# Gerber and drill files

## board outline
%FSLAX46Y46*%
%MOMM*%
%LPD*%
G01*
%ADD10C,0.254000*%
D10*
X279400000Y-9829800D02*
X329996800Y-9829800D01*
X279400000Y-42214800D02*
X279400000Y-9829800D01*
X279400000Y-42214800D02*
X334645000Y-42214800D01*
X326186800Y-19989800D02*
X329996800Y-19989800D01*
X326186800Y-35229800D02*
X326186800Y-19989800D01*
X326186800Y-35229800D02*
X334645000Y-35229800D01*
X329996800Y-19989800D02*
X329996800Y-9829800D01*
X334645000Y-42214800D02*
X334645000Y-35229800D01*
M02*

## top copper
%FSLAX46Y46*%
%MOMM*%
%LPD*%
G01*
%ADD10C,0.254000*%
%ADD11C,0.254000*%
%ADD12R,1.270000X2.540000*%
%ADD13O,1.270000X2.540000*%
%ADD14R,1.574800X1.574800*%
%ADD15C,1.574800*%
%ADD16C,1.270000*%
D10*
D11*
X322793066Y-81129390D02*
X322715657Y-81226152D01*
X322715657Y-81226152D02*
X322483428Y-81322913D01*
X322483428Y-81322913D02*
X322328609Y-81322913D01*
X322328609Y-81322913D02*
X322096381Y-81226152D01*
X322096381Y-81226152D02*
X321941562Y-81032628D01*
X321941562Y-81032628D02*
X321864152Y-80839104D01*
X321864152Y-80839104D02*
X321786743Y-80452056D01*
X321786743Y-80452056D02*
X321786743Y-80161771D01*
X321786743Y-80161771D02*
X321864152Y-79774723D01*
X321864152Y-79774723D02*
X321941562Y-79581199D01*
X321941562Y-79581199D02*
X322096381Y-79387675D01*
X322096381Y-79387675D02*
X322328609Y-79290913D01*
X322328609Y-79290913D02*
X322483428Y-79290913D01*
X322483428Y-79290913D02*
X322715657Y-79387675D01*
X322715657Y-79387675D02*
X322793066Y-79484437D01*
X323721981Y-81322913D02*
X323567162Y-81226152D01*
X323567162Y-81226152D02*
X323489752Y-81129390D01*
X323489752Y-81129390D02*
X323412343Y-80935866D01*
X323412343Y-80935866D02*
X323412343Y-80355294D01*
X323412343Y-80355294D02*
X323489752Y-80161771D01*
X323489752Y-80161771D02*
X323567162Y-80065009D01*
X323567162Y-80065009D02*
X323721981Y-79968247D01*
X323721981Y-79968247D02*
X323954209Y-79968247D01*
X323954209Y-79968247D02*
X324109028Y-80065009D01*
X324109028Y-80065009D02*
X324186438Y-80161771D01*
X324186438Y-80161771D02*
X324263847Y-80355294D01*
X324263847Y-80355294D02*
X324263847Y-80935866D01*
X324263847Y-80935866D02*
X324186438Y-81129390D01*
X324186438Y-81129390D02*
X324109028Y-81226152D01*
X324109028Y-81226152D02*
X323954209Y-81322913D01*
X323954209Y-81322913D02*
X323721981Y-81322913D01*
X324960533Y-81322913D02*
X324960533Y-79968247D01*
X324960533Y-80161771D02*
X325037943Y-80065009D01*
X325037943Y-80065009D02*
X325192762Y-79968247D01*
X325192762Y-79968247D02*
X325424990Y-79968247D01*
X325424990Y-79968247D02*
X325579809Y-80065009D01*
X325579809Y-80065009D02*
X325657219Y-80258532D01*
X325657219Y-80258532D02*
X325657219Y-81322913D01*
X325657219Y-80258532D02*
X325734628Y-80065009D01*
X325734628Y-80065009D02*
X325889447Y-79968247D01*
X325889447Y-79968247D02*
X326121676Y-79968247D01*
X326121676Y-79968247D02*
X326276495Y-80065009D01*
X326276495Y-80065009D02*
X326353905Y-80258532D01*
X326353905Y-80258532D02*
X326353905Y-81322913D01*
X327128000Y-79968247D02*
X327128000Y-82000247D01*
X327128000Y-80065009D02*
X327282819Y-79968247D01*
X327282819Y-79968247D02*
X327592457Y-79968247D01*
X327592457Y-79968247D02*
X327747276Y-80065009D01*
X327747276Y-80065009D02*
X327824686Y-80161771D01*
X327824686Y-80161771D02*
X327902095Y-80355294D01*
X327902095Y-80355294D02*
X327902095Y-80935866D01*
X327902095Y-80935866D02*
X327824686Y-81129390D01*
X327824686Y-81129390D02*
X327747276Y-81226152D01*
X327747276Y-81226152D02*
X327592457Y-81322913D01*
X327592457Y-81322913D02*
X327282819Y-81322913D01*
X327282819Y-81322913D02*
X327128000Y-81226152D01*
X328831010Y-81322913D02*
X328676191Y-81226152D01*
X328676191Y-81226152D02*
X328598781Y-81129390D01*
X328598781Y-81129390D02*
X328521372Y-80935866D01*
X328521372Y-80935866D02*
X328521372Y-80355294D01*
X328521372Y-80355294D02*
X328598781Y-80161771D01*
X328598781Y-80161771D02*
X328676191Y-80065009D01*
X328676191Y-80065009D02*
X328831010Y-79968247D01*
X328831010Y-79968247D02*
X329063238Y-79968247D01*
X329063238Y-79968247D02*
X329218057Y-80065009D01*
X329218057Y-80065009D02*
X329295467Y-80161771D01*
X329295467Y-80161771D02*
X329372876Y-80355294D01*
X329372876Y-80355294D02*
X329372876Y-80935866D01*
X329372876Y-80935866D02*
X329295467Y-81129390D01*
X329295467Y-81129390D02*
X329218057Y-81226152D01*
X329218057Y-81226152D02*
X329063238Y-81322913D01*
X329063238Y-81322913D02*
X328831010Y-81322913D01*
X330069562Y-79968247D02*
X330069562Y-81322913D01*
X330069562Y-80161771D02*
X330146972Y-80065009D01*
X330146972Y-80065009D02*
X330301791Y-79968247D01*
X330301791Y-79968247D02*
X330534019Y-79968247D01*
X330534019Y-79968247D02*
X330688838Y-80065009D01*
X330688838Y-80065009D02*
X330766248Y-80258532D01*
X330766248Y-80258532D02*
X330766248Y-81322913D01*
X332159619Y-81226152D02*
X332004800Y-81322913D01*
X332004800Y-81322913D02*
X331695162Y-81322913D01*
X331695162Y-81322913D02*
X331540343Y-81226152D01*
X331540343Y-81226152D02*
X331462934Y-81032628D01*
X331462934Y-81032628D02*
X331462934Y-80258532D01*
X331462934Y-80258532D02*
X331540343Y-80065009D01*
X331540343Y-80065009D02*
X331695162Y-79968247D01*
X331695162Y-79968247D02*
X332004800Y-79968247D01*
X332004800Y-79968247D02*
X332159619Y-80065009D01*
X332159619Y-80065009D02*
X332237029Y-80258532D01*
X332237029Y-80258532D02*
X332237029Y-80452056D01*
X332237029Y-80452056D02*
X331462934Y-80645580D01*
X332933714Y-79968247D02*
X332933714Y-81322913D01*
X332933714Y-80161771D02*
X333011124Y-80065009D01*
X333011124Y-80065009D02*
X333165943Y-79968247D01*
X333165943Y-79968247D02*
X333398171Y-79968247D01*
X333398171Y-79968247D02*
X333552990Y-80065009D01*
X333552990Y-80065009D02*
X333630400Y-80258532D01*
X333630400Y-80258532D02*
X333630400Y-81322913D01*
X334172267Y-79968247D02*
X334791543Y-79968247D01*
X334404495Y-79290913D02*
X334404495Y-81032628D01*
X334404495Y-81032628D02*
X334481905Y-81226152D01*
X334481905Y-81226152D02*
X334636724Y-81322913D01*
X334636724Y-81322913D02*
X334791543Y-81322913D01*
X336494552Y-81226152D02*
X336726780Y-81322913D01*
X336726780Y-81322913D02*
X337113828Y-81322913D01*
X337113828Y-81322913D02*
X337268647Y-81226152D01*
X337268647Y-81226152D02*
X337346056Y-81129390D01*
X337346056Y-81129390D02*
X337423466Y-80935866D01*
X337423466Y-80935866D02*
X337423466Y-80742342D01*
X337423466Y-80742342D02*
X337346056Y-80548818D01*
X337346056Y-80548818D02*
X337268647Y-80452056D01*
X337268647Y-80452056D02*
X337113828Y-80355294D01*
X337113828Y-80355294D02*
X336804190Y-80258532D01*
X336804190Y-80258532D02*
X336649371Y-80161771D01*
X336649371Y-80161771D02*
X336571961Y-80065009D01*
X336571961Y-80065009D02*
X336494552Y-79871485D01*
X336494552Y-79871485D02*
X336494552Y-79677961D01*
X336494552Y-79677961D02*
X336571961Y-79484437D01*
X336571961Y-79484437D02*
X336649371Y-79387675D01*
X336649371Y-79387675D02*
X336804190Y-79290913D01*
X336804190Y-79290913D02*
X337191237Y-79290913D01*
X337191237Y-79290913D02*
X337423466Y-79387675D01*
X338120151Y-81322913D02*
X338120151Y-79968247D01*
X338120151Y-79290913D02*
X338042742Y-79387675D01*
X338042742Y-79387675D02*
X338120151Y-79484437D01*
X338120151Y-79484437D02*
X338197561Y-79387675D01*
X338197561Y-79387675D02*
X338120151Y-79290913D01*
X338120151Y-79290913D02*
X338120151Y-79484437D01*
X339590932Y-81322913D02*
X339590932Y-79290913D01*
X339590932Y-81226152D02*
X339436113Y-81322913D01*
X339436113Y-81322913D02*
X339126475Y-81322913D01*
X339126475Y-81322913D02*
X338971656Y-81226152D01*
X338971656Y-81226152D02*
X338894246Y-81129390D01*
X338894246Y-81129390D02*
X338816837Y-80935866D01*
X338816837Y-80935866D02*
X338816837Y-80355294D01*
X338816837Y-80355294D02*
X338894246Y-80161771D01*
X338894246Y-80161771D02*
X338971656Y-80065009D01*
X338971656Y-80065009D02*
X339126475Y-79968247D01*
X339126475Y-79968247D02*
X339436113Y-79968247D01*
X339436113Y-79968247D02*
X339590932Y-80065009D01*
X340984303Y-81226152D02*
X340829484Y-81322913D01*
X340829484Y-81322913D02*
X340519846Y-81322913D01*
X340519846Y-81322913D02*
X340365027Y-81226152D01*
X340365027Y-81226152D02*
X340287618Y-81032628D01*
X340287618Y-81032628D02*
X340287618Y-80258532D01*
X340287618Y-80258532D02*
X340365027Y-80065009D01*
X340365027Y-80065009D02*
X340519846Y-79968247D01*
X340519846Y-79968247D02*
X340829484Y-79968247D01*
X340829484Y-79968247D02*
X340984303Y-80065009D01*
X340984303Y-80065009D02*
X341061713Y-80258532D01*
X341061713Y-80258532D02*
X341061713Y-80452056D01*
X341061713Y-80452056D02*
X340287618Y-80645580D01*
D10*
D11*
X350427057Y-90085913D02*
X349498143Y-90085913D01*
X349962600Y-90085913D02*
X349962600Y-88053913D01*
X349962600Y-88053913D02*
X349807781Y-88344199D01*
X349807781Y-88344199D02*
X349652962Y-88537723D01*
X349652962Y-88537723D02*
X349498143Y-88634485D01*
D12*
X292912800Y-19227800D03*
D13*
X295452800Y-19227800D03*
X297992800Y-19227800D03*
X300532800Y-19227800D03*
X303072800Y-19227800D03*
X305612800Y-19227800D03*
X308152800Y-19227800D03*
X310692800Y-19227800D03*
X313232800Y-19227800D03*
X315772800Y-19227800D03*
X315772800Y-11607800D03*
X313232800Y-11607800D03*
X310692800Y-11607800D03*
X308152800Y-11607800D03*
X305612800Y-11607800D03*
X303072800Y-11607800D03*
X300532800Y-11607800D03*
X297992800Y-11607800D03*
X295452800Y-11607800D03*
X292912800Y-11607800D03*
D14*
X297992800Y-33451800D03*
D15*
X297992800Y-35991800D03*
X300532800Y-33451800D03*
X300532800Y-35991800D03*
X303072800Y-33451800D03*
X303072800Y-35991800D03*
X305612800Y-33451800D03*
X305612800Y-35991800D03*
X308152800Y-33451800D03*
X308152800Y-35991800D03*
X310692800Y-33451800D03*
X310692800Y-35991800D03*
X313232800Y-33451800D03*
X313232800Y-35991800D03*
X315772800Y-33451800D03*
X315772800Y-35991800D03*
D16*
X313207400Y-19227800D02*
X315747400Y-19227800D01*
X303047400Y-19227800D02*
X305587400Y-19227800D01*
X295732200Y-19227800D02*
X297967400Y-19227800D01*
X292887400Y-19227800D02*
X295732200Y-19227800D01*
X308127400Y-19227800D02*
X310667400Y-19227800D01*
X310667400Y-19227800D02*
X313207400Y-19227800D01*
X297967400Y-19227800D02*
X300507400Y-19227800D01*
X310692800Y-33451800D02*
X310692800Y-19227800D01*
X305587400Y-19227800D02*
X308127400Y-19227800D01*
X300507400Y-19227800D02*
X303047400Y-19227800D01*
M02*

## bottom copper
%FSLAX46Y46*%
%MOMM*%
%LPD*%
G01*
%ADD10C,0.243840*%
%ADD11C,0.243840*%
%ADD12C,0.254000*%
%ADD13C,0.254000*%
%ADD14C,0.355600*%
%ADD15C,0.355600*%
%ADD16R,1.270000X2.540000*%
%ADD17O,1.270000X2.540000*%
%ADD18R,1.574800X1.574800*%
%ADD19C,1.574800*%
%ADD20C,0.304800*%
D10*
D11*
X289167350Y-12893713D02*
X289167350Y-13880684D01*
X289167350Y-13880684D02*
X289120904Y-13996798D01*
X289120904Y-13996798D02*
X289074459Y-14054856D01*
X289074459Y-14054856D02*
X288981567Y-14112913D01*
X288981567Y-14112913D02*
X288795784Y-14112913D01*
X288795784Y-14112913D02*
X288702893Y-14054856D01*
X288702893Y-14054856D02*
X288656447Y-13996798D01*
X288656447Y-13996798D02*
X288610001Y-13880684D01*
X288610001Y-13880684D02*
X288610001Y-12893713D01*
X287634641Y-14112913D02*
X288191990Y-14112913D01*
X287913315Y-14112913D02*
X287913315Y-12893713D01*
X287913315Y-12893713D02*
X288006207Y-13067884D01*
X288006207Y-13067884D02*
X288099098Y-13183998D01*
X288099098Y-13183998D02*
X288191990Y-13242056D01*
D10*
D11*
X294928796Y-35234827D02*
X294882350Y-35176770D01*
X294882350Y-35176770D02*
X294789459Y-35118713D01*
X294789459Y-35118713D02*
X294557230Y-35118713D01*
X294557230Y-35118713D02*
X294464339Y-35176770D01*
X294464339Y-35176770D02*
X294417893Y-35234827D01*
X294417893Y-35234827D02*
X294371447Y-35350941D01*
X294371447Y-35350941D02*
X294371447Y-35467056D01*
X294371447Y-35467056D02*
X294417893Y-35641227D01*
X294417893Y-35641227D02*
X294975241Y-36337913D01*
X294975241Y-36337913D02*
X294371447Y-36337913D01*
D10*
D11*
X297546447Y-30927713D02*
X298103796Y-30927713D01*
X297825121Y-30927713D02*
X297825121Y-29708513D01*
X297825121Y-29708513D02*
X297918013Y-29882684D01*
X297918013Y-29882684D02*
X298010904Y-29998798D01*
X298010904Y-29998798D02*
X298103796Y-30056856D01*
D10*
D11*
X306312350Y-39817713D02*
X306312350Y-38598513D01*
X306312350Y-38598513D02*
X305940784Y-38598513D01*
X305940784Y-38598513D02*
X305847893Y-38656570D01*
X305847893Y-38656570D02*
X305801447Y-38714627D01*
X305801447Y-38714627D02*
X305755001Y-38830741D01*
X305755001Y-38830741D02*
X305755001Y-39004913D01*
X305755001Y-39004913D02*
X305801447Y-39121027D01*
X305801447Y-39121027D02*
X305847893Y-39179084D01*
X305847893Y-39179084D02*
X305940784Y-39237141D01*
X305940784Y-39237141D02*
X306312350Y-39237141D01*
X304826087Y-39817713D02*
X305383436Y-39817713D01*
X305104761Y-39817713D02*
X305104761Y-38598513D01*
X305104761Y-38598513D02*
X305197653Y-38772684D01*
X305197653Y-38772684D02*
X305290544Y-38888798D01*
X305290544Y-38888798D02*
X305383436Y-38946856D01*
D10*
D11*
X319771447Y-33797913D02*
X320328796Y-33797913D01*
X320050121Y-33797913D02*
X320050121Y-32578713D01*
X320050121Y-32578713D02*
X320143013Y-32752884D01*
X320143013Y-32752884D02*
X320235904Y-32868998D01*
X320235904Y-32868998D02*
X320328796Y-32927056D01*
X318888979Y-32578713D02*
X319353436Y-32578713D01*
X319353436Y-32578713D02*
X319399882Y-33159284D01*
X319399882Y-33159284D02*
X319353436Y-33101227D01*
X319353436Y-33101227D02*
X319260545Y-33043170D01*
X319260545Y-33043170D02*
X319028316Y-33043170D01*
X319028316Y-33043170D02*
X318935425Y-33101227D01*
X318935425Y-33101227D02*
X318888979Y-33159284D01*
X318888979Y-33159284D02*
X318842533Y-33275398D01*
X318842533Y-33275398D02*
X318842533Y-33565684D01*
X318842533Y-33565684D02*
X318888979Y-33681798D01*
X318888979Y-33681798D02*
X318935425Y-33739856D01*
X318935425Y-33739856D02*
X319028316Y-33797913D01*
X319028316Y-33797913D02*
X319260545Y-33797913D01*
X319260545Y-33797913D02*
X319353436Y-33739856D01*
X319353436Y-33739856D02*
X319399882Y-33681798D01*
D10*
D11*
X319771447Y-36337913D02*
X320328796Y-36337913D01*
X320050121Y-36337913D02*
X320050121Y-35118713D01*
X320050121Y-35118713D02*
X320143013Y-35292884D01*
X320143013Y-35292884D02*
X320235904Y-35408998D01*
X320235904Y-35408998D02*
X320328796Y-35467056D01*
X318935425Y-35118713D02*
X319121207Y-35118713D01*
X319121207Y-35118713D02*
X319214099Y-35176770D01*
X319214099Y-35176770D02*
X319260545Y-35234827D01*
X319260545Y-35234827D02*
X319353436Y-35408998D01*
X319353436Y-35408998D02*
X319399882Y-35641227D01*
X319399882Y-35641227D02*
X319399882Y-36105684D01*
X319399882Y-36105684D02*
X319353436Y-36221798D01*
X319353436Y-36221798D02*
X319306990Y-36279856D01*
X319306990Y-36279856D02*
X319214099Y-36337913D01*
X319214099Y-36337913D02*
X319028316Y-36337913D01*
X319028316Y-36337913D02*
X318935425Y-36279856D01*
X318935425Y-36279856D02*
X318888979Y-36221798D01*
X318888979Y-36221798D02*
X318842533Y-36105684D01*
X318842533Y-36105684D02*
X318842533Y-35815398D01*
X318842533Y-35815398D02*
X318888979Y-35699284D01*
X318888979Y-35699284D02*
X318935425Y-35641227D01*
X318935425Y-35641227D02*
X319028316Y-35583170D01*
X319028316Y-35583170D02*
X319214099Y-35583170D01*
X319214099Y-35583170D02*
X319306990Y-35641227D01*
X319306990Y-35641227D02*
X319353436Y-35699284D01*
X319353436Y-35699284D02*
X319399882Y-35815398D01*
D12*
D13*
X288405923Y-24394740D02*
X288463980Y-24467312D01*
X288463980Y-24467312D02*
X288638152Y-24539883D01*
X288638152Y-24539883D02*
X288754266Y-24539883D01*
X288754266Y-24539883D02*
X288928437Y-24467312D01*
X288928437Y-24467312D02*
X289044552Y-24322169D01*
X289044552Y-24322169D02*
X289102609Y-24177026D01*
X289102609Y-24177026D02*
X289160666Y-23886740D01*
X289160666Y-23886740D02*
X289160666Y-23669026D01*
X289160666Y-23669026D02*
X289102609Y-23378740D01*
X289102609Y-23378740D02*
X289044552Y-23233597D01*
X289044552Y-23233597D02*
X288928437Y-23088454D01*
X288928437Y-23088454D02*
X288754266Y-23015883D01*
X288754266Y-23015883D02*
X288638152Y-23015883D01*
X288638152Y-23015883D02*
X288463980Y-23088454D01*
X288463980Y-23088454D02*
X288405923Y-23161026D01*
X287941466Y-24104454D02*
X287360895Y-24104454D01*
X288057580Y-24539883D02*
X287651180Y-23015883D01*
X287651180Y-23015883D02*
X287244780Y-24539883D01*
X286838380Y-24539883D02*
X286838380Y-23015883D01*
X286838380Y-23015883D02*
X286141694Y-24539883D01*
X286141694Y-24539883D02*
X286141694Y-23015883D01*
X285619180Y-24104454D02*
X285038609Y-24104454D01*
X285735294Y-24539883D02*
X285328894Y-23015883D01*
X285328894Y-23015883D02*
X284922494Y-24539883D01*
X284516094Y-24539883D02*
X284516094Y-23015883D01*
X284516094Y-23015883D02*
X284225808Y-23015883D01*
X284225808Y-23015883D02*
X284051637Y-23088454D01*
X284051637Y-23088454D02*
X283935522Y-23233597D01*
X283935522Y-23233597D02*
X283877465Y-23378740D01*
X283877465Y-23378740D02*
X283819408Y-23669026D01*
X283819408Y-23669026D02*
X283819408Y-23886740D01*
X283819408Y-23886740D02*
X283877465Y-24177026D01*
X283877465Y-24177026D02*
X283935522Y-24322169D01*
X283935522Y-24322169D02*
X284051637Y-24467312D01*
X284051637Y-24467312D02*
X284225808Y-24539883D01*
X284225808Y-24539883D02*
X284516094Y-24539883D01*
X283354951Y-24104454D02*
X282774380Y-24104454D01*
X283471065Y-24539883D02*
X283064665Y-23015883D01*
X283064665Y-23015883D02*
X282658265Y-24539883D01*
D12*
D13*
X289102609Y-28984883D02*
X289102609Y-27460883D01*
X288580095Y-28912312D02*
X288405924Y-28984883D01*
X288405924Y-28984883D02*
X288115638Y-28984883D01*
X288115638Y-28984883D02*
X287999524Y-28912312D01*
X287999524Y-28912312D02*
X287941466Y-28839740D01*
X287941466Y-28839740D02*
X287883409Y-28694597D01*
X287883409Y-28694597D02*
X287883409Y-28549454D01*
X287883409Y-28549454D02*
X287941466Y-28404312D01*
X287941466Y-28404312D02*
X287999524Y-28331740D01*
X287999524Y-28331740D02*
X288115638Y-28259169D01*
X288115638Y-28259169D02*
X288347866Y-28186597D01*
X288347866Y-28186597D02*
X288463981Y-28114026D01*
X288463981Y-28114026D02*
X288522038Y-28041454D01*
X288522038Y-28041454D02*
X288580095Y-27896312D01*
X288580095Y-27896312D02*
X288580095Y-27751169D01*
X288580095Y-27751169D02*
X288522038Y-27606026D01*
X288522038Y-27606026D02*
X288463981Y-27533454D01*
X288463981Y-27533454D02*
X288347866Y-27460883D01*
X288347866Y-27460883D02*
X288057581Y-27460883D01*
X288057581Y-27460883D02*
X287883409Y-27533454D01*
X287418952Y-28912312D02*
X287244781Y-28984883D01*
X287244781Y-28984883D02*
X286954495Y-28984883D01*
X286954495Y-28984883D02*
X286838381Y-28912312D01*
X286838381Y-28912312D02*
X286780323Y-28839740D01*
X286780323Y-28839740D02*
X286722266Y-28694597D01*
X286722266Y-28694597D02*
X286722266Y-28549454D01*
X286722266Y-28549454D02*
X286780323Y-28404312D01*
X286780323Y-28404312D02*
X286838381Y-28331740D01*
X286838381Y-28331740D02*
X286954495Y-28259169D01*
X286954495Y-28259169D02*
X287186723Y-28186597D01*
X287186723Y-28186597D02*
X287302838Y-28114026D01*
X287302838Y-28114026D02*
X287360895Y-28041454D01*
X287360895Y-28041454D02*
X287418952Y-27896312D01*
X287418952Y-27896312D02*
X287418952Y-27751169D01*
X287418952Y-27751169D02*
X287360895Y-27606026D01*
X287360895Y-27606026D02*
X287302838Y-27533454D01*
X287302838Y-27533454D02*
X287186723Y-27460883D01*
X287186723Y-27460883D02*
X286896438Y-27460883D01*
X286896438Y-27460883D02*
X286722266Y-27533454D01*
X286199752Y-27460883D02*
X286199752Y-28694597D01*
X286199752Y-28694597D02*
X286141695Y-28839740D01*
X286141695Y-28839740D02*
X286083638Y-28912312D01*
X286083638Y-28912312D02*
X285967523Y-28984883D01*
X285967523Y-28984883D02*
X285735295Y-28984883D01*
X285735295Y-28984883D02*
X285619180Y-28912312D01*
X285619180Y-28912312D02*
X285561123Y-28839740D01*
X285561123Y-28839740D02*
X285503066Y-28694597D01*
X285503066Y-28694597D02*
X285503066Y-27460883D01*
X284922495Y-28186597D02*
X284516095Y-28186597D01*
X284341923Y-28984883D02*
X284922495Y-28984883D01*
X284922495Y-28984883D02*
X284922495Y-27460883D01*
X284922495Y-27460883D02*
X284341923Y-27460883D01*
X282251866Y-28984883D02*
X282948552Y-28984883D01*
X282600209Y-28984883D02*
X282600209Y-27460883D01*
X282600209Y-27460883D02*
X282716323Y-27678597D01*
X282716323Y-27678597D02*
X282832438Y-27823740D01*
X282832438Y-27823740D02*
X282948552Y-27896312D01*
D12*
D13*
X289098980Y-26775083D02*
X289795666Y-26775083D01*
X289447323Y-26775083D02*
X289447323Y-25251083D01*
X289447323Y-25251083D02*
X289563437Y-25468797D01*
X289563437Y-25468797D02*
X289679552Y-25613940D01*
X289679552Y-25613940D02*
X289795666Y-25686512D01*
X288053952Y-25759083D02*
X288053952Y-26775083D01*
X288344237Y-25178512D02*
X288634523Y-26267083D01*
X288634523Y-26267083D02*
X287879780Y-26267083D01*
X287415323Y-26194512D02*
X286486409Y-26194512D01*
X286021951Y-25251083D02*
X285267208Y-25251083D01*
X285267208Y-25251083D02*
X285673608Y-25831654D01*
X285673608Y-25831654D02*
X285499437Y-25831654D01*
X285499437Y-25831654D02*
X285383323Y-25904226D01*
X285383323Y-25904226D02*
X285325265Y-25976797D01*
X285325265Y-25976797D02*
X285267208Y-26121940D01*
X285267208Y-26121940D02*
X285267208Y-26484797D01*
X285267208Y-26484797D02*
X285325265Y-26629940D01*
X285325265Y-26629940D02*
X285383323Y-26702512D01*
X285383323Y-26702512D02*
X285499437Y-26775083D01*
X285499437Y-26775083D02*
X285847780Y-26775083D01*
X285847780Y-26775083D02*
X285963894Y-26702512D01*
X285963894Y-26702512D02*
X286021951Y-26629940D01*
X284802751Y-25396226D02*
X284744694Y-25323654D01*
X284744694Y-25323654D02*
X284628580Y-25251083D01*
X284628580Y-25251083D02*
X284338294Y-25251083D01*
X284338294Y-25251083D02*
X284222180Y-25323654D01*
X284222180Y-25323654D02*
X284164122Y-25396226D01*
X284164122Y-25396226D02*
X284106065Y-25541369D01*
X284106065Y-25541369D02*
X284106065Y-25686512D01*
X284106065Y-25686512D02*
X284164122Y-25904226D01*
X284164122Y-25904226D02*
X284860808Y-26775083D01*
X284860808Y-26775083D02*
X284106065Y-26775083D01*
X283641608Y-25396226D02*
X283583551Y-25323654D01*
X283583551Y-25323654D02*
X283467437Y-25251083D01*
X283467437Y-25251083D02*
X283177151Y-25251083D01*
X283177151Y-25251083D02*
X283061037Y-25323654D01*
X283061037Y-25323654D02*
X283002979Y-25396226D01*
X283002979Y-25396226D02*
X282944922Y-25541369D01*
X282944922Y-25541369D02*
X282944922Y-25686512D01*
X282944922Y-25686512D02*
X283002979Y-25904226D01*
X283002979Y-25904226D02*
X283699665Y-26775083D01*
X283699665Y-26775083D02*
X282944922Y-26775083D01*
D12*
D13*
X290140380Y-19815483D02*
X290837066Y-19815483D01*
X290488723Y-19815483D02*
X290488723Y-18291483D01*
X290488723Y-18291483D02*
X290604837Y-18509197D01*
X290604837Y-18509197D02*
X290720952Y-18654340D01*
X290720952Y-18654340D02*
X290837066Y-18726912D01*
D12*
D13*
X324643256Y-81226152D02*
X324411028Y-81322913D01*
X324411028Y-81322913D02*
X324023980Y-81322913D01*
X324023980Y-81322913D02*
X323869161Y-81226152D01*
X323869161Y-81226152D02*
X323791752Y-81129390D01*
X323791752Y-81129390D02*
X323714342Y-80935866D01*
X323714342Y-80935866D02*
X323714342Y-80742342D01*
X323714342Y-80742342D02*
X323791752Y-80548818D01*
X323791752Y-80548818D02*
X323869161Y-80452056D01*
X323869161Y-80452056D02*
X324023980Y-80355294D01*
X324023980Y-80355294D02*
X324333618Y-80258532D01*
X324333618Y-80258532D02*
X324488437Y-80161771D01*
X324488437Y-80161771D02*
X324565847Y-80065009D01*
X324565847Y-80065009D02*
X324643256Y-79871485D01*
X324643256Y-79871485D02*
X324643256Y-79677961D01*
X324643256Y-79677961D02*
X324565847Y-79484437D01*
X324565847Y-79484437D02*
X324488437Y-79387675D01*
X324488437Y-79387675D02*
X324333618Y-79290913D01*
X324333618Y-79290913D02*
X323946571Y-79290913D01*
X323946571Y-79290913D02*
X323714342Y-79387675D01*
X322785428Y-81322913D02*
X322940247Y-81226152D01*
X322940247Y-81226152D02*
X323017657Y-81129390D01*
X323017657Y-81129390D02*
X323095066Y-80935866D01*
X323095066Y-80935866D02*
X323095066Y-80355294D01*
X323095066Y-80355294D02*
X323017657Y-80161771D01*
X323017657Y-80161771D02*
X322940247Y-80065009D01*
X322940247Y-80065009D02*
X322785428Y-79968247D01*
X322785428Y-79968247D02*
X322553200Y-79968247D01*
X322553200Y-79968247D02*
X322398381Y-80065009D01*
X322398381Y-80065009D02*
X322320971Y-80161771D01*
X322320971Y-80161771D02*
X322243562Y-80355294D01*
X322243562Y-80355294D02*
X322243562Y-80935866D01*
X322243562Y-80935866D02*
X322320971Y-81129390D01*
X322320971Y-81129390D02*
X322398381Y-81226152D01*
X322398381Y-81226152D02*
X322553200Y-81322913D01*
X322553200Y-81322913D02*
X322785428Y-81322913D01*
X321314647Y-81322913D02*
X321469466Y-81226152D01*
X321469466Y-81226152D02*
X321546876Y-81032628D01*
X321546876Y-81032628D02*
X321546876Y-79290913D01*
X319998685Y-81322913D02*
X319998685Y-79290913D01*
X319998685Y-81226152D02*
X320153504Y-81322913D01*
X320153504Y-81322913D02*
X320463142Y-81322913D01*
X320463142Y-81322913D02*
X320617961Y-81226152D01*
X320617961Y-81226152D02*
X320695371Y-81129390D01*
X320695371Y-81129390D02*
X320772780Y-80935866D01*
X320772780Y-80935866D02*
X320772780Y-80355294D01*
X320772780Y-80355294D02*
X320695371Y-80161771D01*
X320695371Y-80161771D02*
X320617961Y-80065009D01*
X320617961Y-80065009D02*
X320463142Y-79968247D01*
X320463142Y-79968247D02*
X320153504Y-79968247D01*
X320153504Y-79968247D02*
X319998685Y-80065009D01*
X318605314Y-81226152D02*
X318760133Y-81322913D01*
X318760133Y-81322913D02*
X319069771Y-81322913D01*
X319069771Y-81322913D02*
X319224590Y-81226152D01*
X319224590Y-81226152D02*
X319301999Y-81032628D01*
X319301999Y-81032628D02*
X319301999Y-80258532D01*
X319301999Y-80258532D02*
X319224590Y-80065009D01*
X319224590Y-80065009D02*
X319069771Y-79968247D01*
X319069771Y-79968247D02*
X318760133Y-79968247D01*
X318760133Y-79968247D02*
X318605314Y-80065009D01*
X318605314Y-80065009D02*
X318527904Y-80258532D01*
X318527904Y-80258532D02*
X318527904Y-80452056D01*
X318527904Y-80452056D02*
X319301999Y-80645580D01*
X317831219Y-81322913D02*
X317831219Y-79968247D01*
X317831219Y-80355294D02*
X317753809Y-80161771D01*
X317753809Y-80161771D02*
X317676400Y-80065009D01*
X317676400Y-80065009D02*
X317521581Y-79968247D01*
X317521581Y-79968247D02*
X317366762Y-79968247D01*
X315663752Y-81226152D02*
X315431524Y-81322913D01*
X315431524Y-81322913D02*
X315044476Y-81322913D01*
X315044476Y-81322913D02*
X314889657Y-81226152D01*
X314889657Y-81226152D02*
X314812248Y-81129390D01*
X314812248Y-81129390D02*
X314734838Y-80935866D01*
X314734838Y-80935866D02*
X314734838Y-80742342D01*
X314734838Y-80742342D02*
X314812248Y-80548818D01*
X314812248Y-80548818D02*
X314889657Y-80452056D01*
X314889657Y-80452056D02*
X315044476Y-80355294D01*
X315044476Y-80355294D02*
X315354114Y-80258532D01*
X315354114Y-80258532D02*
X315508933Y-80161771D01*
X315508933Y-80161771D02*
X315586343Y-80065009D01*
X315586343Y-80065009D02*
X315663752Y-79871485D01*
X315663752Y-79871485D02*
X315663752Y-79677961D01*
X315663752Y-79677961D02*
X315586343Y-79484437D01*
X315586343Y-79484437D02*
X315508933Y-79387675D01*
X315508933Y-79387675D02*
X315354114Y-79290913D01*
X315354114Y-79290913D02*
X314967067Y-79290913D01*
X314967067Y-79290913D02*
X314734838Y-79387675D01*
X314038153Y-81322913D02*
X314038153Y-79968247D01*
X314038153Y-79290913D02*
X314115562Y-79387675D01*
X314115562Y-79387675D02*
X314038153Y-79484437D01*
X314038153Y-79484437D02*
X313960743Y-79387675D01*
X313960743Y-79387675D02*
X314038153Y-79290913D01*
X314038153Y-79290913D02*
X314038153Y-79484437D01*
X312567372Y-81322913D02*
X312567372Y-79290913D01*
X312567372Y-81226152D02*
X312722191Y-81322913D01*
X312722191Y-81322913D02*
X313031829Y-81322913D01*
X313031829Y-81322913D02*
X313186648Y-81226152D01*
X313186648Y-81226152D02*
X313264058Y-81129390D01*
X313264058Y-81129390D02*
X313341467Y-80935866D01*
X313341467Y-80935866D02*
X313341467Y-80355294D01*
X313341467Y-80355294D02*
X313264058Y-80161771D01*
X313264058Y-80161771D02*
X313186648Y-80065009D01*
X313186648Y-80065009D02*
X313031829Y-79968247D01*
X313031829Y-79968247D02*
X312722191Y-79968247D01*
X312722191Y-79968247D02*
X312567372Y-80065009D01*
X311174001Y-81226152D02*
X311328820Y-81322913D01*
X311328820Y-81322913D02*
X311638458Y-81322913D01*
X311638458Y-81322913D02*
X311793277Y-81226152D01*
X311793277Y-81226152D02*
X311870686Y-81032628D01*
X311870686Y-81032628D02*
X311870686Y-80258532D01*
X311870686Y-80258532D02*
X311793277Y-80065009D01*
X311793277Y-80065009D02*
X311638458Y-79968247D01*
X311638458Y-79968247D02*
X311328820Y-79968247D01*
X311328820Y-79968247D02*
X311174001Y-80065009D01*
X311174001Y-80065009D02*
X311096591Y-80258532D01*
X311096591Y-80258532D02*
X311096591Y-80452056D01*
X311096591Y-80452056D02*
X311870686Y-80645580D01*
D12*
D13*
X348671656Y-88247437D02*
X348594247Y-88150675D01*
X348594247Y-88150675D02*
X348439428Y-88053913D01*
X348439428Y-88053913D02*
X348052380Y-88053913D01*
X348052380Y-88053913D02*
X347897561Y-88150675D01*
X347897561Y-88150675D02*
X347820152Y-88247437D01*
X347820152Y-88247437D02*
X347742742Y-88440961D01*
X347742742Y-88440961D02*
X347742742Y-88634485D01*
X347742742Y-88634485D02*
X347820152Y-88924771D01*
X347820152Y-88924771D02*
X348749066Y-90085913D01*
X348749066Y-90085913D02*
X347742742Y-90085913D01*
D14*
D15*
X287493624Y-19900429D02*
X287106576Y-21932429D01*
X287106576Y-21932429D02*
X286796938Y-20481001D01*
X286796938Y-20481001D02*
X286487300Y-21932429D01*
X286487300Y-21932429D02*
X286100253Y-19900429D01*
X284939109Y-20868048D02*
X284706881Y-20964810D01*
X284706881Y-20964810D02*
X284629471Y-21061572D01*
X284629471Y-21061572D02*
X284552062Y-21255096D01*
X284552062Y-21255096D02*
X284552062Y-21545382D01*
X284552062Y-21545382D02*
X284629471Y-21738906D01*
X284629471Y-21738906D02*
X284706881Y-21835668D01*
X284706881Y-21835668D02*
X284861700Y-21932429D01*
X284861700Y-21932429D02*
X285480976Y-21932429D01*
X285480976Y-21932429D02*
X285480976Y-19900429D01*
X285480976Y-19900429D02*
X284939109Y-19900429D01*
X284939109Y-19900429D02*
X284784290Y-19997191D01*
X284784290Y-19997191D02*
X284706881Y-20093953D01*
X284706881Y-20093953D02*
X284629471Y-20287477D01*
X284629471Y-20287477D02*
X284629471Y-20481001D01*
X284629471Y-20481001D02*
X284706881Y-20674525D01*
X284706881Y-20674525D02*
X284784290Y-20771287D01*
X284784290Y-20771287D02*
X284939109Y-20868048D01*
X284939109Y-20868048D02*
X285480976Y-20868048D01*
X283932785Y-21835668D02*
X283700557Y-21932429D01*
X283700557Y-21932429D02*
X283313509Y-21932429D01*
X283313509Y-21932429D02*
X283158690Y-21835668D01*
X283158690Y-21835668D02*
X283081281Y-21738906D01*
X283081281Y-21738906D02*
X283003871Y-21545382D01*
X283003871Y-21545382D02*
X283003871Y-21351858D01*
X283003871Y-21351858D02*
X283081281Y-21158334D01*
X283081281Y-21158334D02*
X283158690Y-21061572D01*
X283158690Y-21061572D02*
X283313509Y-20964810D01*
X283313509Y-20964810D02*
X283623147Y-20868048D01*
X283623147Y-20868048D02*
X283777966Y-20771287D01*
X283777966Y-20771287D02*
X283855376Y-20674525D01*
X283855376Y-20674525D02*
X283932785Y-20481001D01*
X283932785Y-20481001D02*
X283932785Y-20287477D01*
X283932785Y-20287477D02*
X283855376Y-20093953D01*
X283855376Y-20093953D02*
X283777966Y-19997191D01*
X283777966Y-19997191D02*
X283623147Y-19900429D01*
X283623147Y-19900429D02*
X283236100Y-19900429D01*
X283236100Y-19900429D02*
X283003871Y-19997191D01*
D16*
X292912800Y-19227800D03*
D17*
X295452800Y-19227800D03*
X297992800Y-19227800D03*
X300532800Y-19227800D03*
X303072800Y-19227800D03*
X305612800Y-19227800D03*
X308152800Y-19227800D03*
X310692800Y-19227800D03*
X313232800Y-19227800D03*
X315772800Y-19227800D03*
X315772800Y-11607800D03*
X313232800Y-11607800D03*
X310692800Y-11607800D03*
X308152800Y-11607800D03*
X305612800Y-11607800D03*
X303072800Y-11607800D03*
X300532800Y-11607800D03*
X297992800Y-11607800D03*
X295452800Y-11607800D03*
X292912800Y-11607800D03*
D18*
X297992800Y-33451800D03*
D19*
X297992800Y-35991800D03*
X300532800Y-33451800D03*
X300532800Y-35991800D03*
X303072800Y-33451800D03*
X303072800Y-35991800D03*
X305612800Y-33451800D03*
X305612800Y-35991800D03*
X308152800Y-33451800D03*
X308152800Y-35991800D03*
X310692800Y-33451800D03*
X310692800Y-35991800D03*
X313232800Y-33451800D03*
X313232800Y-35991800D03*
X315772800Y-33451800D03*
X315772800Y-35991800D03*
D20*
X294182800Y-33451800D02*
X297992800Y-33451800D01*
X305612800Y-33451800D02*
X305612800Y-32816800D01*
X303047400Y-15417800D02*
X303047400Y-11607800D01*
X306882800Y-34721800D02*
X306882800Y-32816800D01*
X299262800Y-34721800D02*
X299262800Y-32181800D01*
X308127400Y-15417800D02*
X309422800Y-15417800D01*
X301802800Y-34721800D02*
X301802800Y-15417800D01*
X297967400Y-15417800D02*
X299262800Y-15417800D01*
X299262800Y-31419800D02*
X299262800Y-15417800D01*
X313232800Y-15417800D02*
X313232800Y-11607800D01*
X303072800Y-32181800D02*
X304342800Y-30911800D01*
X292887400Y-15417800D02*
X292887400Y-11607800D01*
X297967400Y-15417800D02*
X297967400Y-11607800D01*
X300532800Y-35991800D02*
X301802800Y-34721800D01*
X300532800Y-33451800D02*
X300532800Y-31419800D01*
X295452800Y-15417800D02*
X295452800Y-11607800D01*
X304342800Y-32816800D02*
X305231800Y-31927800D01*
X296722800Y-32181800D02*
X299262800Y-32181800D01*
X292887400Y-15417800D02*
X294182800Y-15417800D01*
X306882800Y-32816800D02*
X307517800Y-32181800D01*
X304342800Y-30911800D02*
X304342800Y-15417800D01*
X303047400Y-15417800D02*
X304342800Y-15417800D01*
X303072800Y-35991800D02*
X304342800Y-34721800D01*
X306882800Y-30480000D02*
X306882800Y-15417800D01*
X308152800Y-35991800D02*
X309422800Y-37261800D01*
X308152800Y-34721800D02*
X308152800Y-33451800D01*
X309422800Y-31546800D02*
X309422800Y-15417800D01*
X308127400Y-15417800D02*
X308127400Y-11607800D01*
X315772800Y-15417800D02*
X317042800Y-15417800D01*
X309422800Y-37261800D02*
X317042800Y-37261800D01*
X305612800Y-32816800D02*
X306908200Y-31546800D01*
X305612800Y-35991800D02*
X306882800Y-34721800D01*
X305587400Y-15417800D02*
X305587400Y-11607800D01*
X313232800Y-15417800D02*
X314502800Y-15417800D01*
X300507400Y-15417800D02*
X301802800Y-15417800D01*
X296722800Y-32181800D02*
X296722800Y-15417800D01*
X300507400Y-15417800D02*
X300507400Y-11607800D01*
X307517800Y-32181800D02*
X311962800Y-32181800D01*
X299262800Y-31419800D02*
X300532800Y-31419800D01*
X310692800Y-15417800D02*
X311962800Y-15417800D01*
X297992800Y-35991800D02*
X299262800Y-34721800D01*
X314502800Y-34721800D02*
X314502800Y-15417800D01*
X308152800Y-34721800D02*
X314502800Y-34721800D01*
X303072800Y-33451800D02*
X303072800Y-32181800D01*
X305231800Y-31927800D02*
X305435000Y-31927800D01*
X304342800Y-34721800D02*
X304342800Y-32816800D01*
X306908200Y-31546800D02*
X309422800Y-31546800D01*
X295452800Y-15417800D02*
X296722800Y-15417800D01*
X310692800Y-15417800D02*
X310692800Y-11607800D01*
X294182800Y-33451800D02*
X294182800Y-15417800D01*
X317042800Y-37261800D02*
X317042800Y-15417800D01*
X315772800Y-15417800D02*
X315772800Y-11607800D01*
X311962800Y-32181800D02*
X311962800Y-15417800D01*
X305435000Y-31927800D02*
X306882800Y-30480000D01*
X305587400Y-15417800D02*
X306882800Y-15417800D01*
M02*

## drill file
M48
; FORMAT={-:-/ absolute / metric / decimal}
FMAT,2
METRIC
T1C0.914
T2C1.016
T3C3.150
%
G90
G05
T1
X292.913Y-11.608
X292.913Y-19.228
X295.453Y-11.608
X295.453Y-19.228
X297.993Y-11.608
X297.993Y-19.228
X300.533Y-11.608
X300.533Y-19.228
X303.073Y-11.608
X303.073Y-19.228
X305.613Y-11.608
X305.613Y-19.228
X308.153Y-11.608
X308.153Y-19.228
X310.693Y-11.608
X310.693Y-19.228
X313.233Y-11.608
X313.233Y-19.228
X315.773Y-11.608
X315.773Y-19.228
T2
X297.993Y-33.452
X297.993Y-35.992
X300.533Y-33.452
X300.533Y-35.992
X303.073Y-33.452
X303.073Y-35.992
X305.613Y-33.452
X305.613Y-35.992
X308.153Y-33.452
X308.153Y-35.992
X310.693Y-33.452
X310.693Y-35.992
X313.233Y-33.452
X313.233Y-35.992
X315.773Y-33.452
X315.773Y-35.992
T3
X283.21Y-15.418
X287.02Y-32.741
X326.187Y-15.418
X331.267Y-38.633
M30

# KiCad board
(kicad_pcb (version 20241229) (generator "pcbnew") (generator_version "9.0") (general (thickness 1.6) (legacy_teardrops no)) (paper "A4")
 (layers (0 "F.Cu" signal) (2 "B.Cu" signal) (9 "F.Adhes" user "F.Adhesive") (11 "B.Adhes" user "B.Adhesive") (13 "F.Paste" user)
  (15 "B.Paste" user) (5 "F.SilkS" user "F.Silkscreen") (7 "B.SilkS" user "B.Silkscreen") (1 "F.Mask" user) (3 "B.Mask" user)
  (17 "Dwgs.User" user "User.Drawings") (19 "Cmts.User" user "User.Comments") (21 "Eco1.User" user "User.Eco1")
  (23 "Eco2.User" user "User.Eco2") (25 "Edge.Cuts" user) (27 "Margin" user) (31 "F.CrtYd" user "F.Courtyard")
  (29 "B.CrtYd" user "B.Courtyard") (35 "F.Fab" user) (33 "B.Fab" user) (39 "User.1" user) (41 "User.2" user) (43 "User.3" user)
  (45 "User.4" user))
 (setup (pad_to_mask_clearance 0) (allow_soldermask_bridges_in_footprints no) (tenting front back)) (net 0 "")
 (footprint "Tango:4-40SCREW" (layer "F.Cu") (at 287.02 32.7406)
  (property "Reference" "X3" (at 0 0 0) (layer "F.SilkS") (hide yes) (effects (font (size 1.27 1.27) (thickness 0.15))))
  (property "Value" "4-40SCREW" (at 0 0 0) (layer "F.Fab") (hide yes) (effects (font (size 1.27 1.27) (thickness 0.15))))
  (pad "" np_thru_hole circle (at 0 0) (size 3.1496 3.1496) (drill 3.1496) (layers "*.Cu" "*.Mask")))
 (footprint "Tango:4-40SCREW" (layer "F.Cu") (at 283.21 15.4178)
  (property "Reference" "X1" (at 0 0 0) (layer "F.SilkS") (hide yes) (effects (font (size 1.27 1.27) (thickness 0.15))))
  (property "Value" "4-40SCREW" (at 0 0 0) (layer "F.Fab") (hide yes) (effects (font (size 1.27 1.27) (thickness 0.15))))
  (pad "" np_thru_hole circle (at 0 0) (size 3.1496 3.1496) (drill 3.1496) (layers "*.Cu" "*.Mask")))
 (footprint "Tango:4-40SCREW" (layer "F.Cu") (at 331.2668 38.6334)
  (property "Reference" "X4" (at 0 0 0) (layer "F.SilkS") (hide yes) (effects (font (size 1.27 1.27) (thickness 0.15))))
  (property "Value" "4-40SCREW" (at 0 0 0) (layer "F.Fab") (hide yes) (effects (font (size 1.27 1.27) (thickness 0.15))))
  (pad "" np_thru_hole circle (at 0 0) (size 3.1496 3.1496) (drill 3.1496) (layers "*.Cu" "*.Mask")))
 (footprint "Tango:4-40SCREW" (layer "F.Cu") (at 326.1868 15.4178)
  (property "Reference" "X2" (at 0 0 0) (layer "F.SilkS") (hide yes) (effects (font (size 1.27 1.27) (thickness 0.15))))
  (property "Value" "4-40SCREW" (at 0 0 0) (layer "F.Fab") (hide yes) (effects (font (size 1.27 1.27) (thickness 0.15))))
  (pad "" np_thru_hole circle (at 0 0) (size 3.1496 3.1496) (drill 3.1496) (layers "*.Cu" "*.Mask")))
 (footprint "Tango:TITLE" (layer "F.Cu") (at 370.84 91.1098)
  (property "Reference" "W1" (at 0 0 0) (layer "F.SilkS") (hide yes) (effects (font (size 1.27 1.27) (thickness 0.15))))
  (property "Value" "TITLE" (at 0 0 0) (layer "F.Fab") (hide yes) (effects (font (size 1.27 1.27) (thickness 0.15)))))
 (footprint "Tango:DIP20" (layer "F.Cu") (at 292.9128 19.2278)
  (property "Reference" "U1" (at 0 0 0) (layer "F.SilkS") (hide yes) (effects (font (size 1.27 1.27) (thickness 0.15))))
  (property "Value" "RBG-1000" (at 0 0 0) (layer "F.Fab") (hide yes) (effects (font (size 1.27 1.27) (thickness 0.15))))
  (pad "1" thru_hole rect (at 0 0) (size 1.27 2.54) (drill 0.9144) (layers "*.Cu" "*.Mask") (remove_unused_layers no)
   (thermal_bridge_angle 45))
  (pad "2" thru_hole oval (at 2.54 0) (size 1.27 2.54) (drill 0.9144) (layers "*.Cu" "*.Mask") (remove_unused_layers no)
   (thermal_bridge_angle 45))
  (pad "3" thru_hole oval (at 5.08 0) (size 1.27 2.54) (drill 0.9144) (layers "*.Cu" "*.Mask") (remove_unused_layers no)
   (thermal_bridge_angle 45))
  (pad "4" thru_hole oval (at 7.62 0) (size 1.27 2.54) (drill 0.9144) (layers "*.Cu" "*.Mask") (remove_unused_layers no)
   (thermal_bridge_angle 45))
  (pad "5" thru_hole oval (at 10.16 0) (size 1.27 2.54) (drill 0.9144) (layers "*.Cu" "*.Mask") (remove_unused_layers no)
   (thermal_bridge_angle 45))
  (pad "6" thru_hole oval (at 12.7 0) (size 1.27 2.54) (drill 0.9144) (layers "*.Cu" "*.Mask") (remove_unused_layers no)
   (thermal_bridge_angle 45))
  (pad "7" thru_hole oval (at 15.24 0) (size 1.27 2.54) (drill 0.9144) (layers "*.Cu" "*.Mask") (remove_unused_layers no)
   (thermal_bridge_angle 45))
  (pad "8" thru_hole oval (at 17.78 0) (size 1.27 2.54) (drill 0.9144) (layers "*.Cu" "*.Mask") (remove_unused_layers no)
   (thermal_bridge_angle 45))
  (pad "9" thru_hole oval (at 20.32 0) (size 1.27 2.54) (drill 0.9144) (layers "*.Cu" "*.Mask") (remove_unused_layers no)
   (thermal_bridge_angle 45))
  (pad "10" thru_hole oval (at 22.86 0) (size 1.27 2.54) (drill 0.9144) (layers "*.Cu" "*.Mask") (remove_unused_layers no)
   (thermal_bridge_angle 45))
  (pad "11" thru_hole oval (at 22.86 -7.62) (size 1.27 2.54) (drill 0.9144) (layers "*.Cu" "*.Mask") (remove_unused_layers no)
   (thermal_bridge_angle 45))
  (pad "12" thru_hole oval (at 20.32 -7.62) (size 1.27 2.54) (drill 0.9144) (layers "*.Cu" "*.Mask") (remove_unused_layers no)
   (thermal_bridge_angle 45))
  (pad "13" thru_hole oval (at 17.78 -7.62) (size 1.27 2.54) (drill 0.9144) (layers "*.Cu" "*.Mask") (remove_unused_layers no)
   (thermal_bridge_angle 45))
  (pad "14" thru_hole oval (at 15.24 -7.62) (size 1.27 2.54) (drill 0.9144) (layers "*.Cu" "*.Mask") (remove_unused_layers no)
   (thermal_bridge_angle 45))
  (pad "15" thru_hole oval (at 12.7 -7.62) (size 1.27 2.54) (drill 0.9144) (layers "*.Cu" "*.Mask") (remove_unused_layers no)
   (thermal_bridge_angle 45))
  (pad "16" thru_hole oval (at 10.16 -7.62) (size 1.27 2.54) (drill 0.9144) (layers "*.Cu" "*.Mask") (remove_unused_layers no)
   (thermal_bridge_angle 45))
  (pad "17" thru_hole oval (at 7.62 -7.62) (size 1.27 2.54) (drill 0.9144) (layers "*.Cu" "*.Mask") (remove_unused_layers no)
   (thermal_bridge_angle 45))
  (pad "18" thru_hole oval (at 5.08 -7.62) (size 1.27 2.54) (drill 0.9144) (layers "*.Cu" "*.Mask") (remove_unused_layers no)
   (thermal_bridge_angle 45))
  (pad "19" thru_hole oval (at 2.54 -7.62) (size 1.27 2.54) (drill 0.9144) (layers "*.Cu" "*.Mask") (remove_unused_layers no)
   (thermal_bridge_angle 45))
  (pad "20" thru_hole oval (at 0 -7.62) (size 1.27 2.54) (drill 0.9144) (layers "*.Cu" "*.Mask") (remove_unused_layers no)
   (thermal_bridge_angle 45)))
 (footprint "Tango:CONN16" (layer "F.Cu") (at 297.9928 35.9918)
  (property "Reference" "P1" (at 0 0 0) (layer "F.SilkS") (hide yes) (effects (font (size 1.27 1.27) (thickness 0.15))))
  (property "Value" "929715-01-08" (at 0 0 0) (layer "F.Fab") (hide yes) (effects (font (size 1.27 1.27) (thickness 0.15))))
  (pad "1" thru_hole rect (at 0 -2.54) (size 1.5748 1.5748) (drill 1.016) (layers "*.Cu" "*.Mask") (remove_unused_layers no)
   (thermal_bridge_angle 45))
  (pad "2" thru_hole circle (at 0 0) (size 1.5748 1.5748) (drill 1.016) (layers "*.Cu" "*.Mask") (remove_unused_layers no))
  (pad "3" thru_hole circle (at 2.54 -2.54) (size 1.5748 1.5748) (drill 1.016) (layers "*.Cu" "*.Mask") (remove_unused_layers no))
  (pad "4" thru_hole circle (at 2.54 0) (size 1.5748 1.5748) (drill 1.016) (layers "*.Cu" "*.Mask") (remove_unused_layers no))
  (pad "5" thru_hole circle (at 5.08 -2.54) (size 1.5748 1.5748) (drill 1.016) (layers "*.Cu" "*.Mask") (remove_unused_layers no))
  (pad "6" thru_hole circle (at 5.08 0) (size 1.5748 1.5748) (drill 1.016) (layers "*.Cu" "*.Mask") (remove_unused_layers no))
  (pad "7" thru_hole circle (at 7.62 -2.54) (size 1.5748 1.5748) (drill 1.016) (layers "*.Cu" "*.Mask") (remove_unused_layers no))
  (pad "8" thru_hole circle (at 7.62 0) (size 1.5748 1.5748) (drill 1.016) (layers "*.Cu" "*.Mask") (remove_unused_layers no))
  (pad "9" thru_hole circle (at 10.16 -2.54) (size 1.5748 1.5748) (drill 1.016) (layers "*.Cu" "*.Mask") (remove_unused_layers no))
  (pad "10" thru_hole circle (at 10.16 0) (size 1.5748 1.5748) (drill 1.016) (layers "*.Cu" "*.Mask") (remove_unused_layers no))
  (pad "11" thru_hole circle (at 12.7 -2.54) (size 1.5748 1.5748) (drill 1.016) (layers "*.Cu" "*.Mask") (remove_unused_layers no))
  (pad "12" thru_hole circle (at 12.7 0) (size 1.5748 1.5748) (drill 1.016) (layers "*.Cu" "*.Mask") (remove_unused_layers no))
  (pad "13" thru_hole circle (at 15.24 -2.54) (size 1.5748 1.5748) (drill 1.016) (layers "*.Cu" "*.Mask") (remove_unused_layers no))
  (pad "14" thru_hole circle (at 15.24 0) (size 1.5748 1.5748) (drill 1.016) (layers "*.Cu" "*.Mask") (remove_unused_layers no))
  (pad "15" thru_hole circle (at 17.78 -2.54) (size 1.5748 1.5748) (drill 1.016) (layers "*.Cu" "*.Mask") (remove_unused_layers no))
  (pad "16" thru_hole circle (at 17.78 0) (size 1.5748 1.5748) (drill 1.016) (layers "*.Cu" "*.Mask") (remove_unused_layers no)))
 (gr_line (start 279.4 9.8298) (end 329.9968 9.8298) (stroke (width 0.254) (type default)) (layer "Edge.Cuts"))
 (gr_line (start 279.4 42.2148) (end 279.4 9.8298) (stroke (width 0.254) (type default)) (layer "Edge.Cuts"))
 (gr_line (start 279.4 42.2148) (end 334.645 42.2148) (stroke (width 0.254) (type default)) (layer "Edge.Cuts"))
 (gr_line (start 326.1868 19.9898) (end 329.9968 19.9898) (stroke (width 0.254) (type default)) (layer "Edge.Cuts"))
 (gr_line (start 326.1868 35.2298) (end 326.1868 19.9898) (stroke (width 0.254) (type default)) (layer "Edge.Cuts"))
 (gr_line (start 326.1868 35.2298) (end 334.645 35.2298) (stroke (width 0.254) (type default)) (layer "Edge.Cuts"))
 (gr_line (start 329.9968 19.9898) (end 329.9968 9.8298) (stroke (width 0.254) (type default)) (layer "Edge.Cuts"))
 (gr_line (start 334.645 42.2148) (end 334.645 35.2298) (stroke (width 0.254) (type default)) (layer "Edge.Cuts"))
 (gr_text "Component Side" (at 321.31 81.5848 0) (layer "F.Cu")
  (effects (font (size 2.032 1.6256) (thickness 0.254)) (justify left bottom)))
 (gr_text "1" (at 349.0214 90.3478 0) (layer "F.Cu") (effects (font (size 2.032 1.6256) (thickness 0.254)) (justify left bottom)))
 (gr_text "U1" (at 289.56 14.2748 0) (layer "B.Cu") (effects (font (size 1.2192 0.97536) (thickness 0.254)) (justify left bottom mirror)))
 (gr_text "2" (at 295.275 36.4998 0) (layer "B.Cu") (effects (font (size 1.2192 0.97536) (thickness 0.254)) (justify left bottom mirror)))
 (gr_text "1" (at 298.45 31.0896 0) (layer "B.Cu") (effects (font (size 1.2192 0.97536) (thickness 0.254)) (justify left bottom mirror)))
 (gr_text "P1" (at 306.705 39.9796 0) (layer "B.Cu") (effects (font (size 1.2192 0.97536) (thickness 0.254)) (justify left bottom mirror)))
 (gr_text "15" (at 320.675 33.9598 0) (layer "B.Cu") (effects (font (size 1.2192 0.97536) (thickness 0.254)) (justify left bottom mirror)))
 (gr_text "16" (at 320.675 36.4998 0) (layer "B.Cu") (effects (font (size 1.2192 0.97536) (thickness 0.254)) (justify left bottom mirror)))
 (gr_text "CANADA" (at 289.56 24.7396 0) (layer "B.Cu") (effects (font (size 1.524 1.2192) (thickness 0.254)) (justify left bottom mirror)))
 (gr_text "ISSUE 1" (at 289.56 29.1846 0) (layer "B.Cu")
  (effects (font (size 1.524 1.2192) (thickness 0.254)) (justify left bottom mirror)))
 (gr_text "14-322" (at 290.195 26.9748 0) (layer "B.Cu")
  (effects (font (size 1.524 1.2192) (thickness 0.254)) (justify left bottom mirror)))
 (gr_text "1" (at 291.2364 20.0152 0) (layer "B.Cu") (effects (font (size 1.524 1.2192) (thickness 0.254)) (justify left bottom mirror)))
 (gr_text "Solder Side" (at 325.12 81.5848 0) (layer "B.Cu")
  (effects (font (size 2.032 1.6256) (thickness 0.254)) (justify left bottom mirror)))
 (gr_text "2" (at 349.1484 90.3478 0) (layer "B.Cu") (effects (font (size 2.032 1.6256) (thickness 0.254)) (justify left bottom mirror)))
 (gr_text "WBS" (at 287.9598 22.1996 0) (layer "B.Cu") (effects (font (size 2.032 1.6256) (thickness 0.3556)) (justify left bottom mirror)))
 (segment (start 313.2074 19.2278) (end 315.7474 19.2278) (width 1.27) (layer "F.Cu") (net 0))
 (segment (start 303.0474 19.2278) (end 305.5874 19.2278) (width 1.27) (layer "F.Cu") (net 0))
 (segment (start 295.7322 19.2278) (end 297.9674 19.2278) (width 1.27) (layer "F.Cu") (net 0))
 (segment (start 292.8874 19.2278) (end 295.7322 19.2278) (width 1.27) (layer "F.Cu") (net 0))
 (segment (start 308.1274 19.2278) (end 310.6674 19.2278) (width 1.27) (layer "F.Cu") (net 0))
 (segment (start 310.6674 19.2278) (end 313.2074 19.2278) (width 1.27) (layer "F.Cu") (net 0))
 (segment (start 297.9674 19.2278) (end 300.5074 19.2278) (width 1.27) (layer "F.Cu") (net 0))
 (segment (start 310.6928 33.4518) (end 310.6928 19.2278) (width 1.27) (layer "F.Cu") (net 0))
 (segment (start 305.5874 19.2278) (end 308.1274 19.2278) (width 1.27) (layer "F.Cu") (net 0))
 (segment (start 300.5074 19.2278) (end 303.0474 19.2278) (width 1.27) (layer "F.Cu") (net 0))
 (segment (start 294.1828 33.4518) (end 297.9928 33.4518) (width 0.3048) (layer "B.Cu") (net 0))
 (segment (start 305.6128 33.4518) (end 305.6128 32.8168) (width 0.3048) (layer "B.Cu") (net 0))
 (segment (start 303.0474 15.4178) (end 303.0474 11.6078) (width 0.3048) (layer "B.Cu") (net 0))
 (segment (start 306.8828 34.7218) (end 306.8828 32.8168) (width 0.3048) (layer "B.Cu") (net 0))
 (segment (start 299.2628 34.7218) (end 299.2628 32.1818) (width 0.3048) (layer "B.Cu") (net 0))
 (segment (start 308.1274 15.4178) (end 309.4228 15.4178) (width 0.3048) (layer "B.Cu") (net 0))
 (segment (start 301.8028 34.7218) (end 301.8028 15.4178) (width 0.3048) (layer "B.Cu") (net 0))
 (segment (start 297.9674 15.4178) (end 299.2628 15.4178) (width 0.3048) (layer "B.Cu") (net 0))
 (segment (start 299.2628 31.4198) (end 299.2628 15.4178) (width 0.3048) (layer "B.Cu") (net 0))
 (segment (start 313.2328 15.4178) (end 313.2328 11.6078) (width 0.3048) (layer "B.Cu") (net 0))
 (segment (start 303.0728 32.1818) (end 304.3428 30.9118) (width 0.3048) (layer "B.Cu") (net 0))
 (segment (start 292.8874 15.4178) (end 292.8874 11.6078) (width 0.3048) (layer "B.Cu") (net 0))
 (segment (start 297.9674 15.4178) (end 297.9674 11.6078) (width 0.3048) (layer "B.Cu") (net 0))
 (segment (start 300.5328 35.9918) (end 301.8028 34.7218) (width 0.3048) (layer "B.Cu") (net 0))
 (segment (start 300.5328 33.4518) (end 300.5328 31.4198) (width 0.3048) (layer "B.Cu") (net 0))
 (segment (start 295.4528 15.4178) (end 295.4528 11.6078) (width 0.3048) (layer "B.Cu") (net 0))
 (segment (start 304.3428 32.8168) (end 305.2318 31.9278) (width 0.3048) (layer "B.Cu") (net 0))
 (segment (start 296.7228 32.1818) (end 299.2628 32.1818) (width 0.3048) (layer "B.Cu") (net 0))
 (segment (start 292.8874 15.4178) (end 294.1828 15.4178) (width 0.3048) (layer "B.Cu") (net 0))
 (segment (start 306.8828 32.8168) (end 307.5178 32.1818) (width 0.3048) (layer "B.Cu") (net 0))
 (segment (start 304.3428 30.9118) (end 304.3428 15.4178) (width 0.3048) (layer "B.Cu") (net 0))
 (segment (start 303.0474 15.4178) (end 304.3428 15.4178) (width 0.3048) (layer "B.Cu") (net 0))
 (segment (start 303.0728 35.9918) (end 304.3428 34.7218) (width 0.3048) (layer "B.Cu") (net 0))
 (segment (start 306.8828 30.48) (end 306.8828 15.4178) (width 0.3048) (layer "B.Cu") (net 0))
 (segment (start 308.1528 35.9918) (end 309.4228 37.2618) (width 0.3048) (layer "B.Cu") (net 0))
 (segment (start 308.1528 34.7218) (end 308.1528 33.4518) (width 0.3048) (layer "B.Cu") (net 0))
 (segment (start 309.4228 31.5468) (end 309.4228 15.4178) (width 0.3048) (layer "B.Cu") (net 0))
 (segment (start 308.1274 15.4178) (end 308.1274 11.6078) (width 0.3048) (layer "B.Cu") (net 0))
 (segment (start 315.7728 15.4178) (end 317.0428 15.4178) (width 0.3048) (layer "B.Cu") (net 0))
 (segment (start 309.4228 37.2618) (end 317.0428 37.2618) (width 0.3048) (layer "B.Cu") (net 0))
 (segment (start 305.6128 32.8168) (end 306.9082 31.5468) (width 0.3048) (layer "B.Cu") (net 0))
 (segment (start 305.6128 35.9918) (end 306.8828 34.7218) (width 0.3048) (layer "B.Cu") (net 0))
 (segment (start 305.5874 15.4178) (end 305.5874 11.6078) (width 0.3048) (layer "B.Cu") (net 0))
 (segment (start 313.2328 15.4178) (end 314.5028 15.4178) (width 0.3048) (layer "B.Cu") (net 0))
 (segment (start 300.5074 15.4178) (end 301.8028 15.4178) (width 0.3048) (layer "B.Cu") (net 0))
 (segment (start 296.7228 32.1818) (end 296.7228 15.4178) (width 0.3048) (layer "B.Cu") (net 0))
 (segment (start 300.5074 15.4178) (end 300.5074 11.6078) (width 0.3048) (layer "B.Cu") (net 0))
 (segment (start 307.5178 32.1818) (end 311.9628 32.1818) (width 0.3048) (layer "B.Cu") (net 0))
 (segment (start 299.2628 31.4198) (end 300.5328 31.4198) (width 0.3048) (layer "B.Cu") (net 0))
 (segment (start 310.6928 15.4178) (end 311.9628 15.4178) (width 0.3048) (layer "B.Cu") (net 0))
 (segment (start 297.9928 35.9918) (end 299.2628 34.7218) (width 0.3048) (layer "B.Cu") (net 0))
 (segment (start 314.5028 34.7218) (end 314.5028 15.4178) (width 0.3048) (layer "B.Cu") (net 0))
 (segment (start 308.1528 34.7218) (end 314.5028 34.7218) (width 0.3048) (layer "B.Cu") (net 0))
 (segment (start 303.0728 33.4518) (end 303.0728 32.1818) (width 0.3048) (layer "B.Cu") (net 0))
 (segment (start 305.2318 31.9278) (end 305.435 31.9278) (width 0.3048) (layer "B.Cu") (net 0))
 (segment (start 304.3428 34.7218) (end 304.3428 32.8168) (width 0.3048) (layer "B.Cu") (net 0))
 (segment (start 306.9082 31.5468) (end 309.4228 31.5468) (width 0.3048) (layer "B.Cu") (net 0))
 (segment (start 295.4528 15.4178) (end 296.7228 15.4178) (width 0.3048) (layer "B.Cu") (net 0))
 (segment (start 310.6928 15.4178) (end 310.6928 11.6078) (width 0.3048) (layer "B.Cu") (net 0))
 (segment (start 294.1828 33.4518) (end 294.1828 15.4178) (width 0.3048) (layer "B.Cu") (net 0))
 (segment (start 317.0428 37.2618) (end 317.0428 15.4178) (width 0.3048) (layer "B.Cu") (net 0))
 (segment (start 315.7728 15.4178) (end 315.7728 11.6078) (width 0.3048) (layer "B.Cu") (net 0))
 (segment (start 311.9628 32.1818) (end 311.9628 15.4178) (width 0.3048) (layer "B.Cu") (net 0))
 (segment (start 305.435 31.9278) (end 306.8828 30.48) (width 0.3048) (layer "B.Cu") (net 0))
 (segment (start 305.5874 15.4178) (end 306.8828 15.4178) (width 0.3048) (layer "B.Cu") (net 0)))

